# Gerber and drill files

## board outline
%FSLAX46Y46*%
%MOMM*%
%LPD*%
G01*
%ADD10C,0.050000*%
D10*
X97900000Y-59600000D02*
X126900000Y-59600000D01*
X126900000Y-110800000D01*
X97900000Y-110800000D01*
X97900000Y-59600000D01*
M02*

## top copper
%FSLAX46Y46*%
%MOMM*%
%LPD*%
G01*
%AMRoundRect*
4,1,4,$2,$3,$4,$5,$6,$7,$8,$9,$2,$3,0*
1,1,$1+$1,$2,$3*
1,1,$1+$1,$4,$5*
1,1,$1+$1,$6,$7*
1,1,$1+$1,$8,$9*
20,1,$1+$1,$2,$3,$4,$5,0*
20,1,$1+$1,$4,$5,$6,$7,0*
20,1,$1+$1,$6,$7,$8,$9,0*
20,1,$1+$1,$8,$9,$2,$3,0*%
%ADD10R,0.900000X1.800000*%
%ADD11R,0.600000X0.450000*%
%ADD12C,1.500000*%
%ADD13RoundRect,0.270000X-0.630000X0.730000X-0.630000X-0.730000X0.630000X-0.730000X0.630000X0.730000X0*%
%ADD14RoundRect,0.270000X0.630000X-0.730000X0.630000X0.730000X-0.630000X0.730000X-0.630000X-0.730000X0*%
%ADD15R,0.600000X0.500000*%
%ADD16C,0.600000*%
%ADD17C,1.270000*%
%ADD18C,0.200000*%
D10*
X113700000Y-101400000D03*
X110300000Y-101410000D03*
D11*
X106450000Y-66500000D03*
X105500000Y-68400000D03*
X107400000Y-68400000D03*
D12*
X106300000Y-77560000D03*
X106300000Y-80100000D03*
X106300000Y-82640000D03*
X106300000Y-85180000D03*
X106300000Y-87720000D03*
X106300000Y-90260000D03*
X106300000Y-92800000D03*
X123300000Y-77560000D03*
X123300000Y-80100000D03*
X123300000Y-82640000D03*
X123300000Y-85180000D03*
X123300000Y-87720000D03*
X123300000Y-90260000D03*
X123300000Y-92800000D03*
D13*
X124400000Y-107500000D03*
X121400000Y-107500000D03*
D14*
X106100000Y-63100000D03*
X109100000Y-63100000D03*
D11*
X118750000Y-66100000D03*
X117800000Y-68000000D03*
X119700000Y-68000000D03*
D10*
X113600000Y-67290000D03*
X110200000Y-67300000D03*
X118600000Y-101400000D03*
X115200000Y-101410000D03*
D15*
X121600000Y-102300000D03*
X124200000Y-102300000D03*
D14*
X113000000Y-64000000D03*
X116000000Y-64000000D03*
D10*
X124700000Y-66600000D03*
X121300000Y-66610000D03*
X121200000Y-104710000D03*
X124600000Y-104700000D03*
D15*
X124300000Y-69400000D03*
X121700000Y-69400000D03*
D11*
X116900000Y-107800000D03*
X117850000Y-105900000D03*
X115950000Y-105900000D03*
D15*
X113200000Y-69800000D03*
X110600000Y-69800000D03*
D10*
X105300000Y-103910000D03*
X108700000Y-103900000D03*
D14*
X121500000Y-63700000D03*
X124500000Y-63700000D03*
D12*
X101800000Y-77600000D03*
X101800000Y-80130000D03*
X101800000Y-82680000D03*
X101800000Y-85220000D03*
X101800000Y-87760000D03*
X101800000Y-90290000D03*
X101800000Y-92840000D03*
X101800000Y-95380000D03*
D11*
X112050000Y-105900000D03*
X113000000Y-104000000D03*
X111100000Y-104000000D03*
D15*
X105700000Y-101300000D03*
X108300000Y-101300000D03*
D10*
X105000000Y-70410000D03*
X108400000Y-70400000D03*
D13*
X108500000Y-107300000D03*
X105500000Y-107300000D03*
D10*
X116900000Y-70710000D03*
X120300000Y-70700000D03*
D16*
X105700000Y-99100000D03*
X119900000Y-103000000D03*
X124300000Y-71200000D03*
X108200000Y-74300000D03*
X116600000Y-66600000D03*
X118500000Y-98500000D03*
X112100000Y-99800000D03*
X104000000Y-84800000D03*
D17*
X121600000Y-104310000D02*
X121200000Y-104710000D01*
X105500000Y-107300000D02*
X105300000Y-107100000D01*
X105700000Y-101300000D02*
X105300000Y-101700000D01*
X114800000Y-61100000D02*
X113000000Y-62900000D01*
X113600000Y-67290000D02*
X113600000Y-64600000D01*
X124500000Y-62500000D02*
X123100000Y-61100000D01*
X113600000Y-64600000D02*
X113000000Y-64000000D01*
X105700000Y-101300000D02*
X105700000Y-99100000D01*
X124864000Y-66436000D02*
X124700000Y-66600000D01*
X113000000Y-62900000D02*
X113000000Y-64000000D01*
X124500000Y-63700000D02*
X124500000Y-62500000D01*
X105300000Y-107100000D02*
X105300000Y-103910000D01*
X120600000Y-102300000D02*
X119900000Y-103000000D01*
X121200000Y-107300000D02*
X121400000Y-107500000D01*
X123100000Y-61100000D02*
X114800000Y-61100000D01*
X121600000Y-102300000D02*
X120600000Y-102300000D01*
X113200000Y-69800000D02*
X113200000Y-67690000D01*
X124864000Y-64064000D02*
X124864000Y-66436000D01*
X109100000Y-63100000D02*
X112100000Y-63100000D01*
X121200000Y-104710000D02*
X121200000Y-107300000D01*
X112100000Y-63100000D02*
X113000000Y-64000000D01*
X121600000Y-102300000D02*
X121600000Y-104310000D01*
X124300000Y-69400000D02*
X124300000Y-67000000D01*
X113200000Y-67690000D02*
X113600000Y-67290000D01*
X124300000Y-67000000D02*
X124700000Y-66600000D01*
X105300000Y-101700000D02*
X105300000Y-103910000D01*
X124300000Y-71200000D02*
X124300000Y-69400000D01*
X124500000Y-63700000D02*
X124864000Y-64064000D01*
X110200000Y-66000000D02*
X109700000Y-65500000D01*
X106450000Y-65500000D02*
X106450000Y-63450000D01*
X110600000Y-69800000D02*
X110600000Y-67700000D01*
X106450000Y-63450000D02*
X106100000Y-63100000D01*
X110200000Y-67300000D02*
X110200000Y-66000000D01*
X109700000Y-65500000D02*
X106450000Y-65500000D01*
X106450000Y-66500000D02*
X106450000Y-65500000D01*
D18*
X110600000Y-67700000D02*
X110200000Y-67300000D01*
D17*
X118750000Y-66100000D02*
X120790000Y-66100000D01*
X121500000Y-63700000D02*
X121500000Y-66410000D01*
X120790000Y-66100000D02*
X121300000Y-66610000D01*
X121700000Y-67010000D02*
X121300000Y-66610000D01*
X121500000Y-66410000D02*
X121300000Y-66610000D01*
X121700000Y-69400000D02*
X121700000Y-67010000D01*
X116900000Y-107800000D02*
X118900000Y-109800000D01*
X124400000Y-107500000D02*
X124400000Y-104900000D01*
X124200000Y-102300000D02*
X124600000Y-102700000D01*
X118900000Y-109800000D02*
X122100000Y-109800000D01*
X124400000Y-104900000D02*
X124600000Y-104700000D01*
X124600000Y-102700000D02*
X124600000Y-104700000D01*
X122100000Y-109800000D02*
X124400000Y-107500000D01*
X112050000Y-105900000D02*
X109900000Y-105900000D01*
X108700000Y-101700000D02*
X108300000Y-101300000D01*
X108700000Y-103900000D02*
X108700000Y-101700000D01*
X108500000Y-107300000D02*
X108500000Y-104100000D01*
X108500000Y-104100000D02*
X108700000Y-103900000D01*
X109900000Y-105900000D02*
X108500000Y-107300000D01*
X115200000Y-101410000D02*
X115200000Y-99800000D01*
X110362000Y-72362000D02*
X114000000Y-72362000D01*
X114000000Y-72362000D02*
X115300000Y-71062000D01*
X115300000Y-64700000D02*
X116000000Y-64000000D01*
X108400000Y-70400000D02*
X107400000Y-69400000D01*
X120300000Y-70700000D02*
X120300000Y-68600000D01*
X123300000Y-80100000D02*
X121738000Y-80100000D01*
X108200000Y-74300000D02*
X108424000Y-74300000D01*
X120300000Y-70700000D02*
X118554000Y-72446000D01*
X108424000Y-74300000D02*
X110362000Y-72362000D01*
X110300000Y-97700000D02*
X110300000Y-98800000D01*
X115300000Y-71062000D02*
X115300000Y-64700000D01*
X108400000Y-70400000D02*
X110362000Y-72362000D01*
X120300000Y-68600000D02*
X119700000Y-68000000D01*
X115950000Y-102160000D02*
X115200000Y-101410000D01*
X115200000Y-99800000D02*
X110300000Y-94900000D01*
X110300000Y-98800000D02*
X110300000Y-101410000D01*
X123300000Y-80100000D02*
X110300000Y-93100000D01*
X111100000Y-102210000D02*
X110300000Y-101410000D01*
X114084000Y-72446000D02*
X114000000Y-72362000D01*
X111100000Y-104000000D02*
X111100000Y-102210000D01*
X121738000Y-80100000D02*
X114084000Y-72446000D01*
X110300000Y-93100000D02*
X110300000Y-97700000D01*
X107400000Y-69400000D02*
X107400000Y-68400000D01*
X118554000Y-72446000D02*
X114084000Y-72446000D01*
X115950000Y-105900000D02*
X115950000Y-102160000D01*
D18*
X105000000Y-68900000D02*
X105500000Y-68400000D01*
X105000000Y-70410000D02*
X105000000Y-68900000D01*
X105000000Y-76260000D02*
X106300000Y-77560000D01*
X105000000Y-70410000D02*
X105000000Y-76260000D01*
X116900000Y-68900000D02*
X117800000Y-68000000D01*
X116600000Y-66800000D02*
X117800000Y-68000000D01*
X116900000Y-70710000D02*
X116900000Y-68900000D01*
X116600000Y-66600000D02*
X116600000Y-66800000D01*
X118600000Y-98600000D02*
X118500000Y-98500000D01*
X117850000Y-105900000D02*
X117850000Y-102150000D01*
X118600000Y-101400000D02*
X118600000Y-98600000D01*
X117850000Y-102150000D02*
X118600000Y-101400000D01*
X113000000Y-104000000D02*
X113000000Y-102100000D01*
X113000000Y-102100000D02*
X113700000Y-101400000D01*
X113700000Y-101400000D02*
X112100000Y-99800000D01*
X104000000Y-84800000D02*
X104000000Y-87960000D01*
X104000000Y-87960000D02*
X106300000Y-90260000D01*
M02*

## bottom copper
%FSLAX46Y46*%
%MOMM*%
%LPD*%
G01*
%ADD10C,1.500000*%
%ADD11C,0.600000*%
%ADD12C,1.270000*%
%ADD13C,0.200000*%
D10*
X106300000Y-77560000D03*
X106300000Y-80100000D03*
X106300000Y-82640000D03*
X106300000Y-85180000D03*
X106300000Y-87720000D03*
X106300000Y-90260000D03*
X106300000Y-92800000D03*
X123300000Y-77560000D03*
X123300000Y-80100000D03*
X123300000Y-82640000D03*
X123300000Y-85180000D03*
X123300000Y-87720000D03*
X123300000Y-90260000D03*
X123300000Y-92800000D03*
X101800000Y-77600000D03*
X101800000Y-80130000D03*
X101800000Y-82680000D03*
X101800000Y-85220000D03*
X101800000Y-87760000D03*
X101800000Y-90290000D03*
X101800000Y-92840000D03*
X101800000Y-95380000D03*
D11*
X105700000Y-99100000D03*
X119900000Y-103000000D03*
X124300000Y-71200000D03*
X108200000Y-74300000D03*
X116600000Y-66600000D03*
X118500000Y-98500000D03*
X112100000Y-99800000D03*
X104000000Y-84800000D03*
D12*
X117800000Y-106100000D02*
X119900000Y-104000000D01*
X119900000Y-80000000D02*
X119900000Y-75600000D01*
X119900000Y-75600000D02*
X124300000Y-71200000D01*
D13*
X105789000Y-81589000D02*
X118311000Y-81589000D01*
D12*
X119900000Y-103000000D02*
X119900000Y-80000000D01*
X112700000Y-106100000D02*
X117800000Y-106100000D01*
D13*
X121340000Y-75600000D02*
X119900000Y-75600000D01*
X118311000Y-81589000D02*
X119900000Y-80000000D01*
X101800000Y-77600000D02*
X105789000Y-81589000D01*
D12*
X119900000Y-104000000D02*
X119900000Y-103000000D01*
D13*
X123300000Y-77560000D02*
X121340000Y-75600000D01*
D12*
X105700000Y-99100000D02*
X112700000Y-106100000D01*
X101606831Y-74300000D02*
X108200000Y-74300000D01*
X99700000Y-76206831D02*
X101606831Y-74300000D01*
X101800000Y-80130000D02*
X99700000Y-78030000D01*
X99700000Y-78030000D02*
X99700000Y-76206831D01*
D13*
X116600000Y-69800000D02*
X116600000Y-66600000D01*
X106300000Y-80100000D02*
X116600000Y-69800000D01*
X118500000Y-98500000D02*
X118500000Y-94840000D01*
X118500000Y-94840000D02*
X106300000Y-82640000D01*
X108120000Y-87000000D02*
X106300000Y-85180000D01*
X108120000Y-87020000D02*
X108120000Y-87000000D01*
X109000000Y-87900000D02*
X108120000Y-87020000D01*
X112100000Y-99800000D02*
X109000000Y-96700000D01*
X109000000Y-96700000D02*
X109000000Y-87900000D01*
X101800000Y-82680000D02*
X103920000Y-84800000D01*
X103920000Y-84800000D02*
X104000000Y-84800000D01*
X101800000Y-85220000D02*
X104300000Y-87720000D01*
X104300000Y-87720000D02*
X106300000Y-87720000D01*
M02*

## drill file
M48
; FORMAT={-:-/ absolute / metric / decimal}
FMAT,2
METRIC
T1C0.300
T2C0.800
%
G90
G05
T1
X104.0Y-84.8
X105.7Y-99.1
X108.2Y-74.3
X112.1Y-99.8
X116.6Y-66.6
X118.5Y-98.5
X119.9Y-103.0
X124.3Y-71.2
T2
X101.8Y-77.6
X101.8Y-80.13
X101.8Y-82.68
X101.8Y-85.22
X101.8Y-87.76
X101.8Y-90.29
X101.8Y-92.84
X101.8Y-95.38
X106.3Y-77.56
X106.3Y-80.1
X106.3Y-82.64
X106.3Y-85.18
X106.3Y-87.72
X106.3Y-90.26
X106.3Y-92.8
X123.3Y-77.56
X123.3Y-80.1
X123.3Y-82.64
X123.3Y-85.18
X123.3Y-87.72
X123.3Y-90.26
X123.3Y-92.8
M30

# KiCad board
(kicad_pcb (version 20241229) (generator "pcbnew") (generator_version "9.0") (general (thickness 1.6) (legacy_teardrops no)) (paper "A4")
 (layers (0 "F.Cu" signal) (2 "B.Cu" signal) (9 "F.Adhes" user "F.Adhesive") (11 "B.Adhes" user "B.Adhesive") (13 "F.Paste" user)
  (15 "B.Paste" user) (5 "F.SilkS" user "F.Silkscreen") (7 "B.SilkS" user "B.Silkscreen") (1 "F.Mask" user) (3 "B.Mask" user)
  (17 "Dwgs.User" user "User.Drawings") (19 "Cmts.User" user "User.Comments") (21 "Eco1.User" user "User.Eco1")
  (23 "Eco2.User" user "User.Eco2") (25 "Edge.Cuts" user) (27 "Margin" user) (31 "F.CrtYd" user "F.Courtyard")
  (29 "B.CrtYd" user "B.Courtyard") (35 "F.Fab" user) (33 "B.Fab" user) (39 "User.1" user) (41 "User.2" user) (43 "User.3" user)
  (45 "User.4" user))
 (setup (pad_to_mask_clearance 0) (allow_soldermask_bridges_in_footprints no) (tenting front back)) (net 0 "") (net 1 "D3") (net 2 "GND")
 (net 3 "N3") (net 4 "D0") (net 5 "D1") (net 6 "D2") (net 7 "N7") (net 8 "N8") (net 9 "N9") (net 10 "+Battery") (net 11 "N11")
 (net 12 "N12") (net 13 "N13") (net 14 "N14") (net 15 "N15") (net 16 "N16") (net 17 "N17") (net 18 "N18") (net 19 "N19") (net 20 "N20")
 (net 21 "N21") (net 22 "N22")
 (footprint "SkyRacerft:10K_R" (layer "F.Cu") (at 112 101.41 180)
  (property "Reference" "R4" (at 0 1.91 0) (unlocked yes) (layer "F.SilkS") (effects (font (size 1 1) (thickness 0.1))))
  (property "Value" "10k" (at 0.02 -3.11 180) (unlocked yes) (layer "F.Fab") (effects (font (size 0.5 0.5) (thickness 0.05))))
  (pad "1" smd rect (at -1.7 0.01 180) (size 0.9 1.8) (layers "F.Cu" "F.Mask" "F.Paste") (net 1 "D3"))
  (pad "2" smd rect (at 1.7 0 180) (size 0.9 1.8) (layers "F.Cu" "F.Mask" "F.Paste") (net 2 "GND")))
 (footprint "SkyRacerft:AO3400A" (layer "F.Cu") (at 106.45 67.45)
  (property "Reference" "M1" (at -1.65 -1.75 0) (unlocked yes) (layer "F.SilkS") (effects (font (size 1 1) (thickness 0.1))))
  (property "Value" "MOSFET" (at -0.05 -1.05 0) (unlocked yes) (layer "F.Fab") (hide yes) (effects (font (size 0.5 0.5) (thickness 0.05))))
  (pad "1" smd rect (at 0 -0.95 90) (size 0.45 0.6) (layers "F.Cu" "F.Mask" "F.Paste") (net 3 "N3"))
  (pad "2" smd rect (at -0.95 0.95 90) (size 0.45 0.6) (layers "F.Cu" "F.Mask" "F.Paste") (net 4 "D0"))
  (pad "3" smd rect (at 0.95 0.95 90) (size 0.45 0.6) (layers "F.Cu" "F.Mask" "F.Paste") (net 2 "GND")))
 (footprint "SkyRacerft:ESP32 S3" (layer "F.Cu") (at 114.8 77.56)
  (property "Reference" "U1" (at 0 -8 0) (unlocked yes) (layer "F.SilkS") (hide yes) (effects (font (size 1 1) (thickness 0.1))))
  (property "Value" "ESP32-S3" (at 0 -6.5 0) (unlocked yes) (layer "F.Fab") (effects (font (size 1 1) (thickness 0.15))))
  (pad "1" thru_hole circle (at -8.5 0) (size 1.5 1.5) (drill 0.8) (layers "*.Cu" "*.Mask") (remove_unused_layers no) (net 4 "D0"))
  (pad "2" thru_hole circle (at -8.5 2.54) (size 1.5 1.5) (drill 0.8) (layers "*.Cu" "*.Mask") (remove_unused_layers no) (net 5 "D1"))
  (pad "3" thru_hole circle (at -8.5 5.08) (size 1.5 1.5) (drill 0.8) (layers "*.Cu" "*.Mask") (remove_unused_layers no) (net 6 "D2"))
  (pad "4" thru_hole circle (at -8.5 7.62) (size 1.5 1.5) (drill 0.8) (layers "*.Cu" "*.Mask") (remove_unused_layers no) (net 1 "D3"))
  (pad "5" thru_hole circle (at -8.5 10.16) (size 1.5 1.5) (drill 0.8) (layers "*.Cu" "*.Mask") (remove_unused_layers no) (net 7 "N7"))
  (pad "6" thru_hole circle (at -8.5 12.7) (size 1.5 1.5) (drill 0.8) (layers "*.Cu" "*.Mask") (remove_unused_layers no) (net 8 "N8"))
  (pad "7" thru_hole circle (at -8.5 15.24) (size 1.5 1.5) (drill 0.8) (layers "*.Cu" "*.Mask") (remove_unused_layers no) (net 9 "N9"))
  (pad "8" thru_hole circle (at 8.5 0) (size 1.5 1.5) (drill 0.8) (layers "*.Cu" "*.Mask") (remove_unused_layers no) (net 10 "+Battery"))
  (pad "9" thru_hole circle (at 8.5 2.54) (size 1.5 1.5) (drill 0.8) (layers "*.Cu" "*.Mask") (remove_unused_layers no) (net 2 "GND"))
  (pad "10" thru_hole circle (at 8.5 5.08) (size 1.5 1.5) (drill 0.8) (layers "*.Cu" "*.Mask") (remove_unused_layers no) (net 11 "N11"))
  (pad "11" thru_hole circle (at 8.5 7.62) (size 1.5 1.5) (drill 0.8) (layers "*.Cu" "*.Mask") (remove_unused_layers no) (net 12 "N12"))
  (pad "12" thru_hole circle (at 8.5 10.16) (size 1.5 1.5) (drill 0.8) (layers "*.Cu" "*.Mask") (remove_unused_layers no) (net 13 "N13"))
  (pad "13" thru_hole circle (at 8.5 12.7) (size 1.5 1.5) (drill 0.8) (layers "*.Cu" "*.Mask") (remove_unused_layers no) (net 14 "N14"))
  (pad "14" thru_hole circle (at 8.5 15.24) (size 1.5 1.5) (drill 0.8) (layers "*.Cu" "*.Mask") (remove_unused_layers no) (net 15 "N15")))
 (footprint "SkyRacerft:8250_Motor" (layer "F.Cu") (at 122.9 107.5 180)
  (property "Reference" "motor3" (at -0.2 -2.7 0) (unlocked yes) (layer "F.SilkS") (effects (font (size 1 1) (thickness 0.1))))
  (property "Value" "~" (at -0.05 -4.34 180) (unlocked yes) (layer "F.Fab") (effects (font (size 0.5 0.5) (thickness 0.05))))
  (pad "1" smd roundrect (at -1.5 0 270) (size 2 1.8) (layers "F.Cu" "F.Mask" "F.Paste") (roundrect_rratio 0.15) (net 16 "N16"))
  (pad "2" smd roundrect (at 1.5 0 270) (size 2 1.8) (layers "F.Cu" "F.Mask" "F.Paste") (roundrect_rratio 0.15) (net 10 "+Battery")))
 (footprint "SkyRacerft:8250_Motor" (layer "F.Cu") (at 107.6 63.1)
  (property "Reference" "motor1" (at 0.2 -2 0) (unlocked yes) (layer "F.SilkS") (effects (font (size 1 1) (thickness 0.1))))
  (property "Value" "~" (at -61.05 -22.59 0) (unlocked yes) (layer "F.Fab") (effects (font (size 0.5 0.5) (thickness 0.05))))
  (pad "1" smd roundrect (at -1.5 0 90) (size 2 1.8) (layers "F.Cu" "F.Mask" "F.Paste") (roundrect_rratio 0.15) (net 3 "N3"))
  (pad "2" smd roundrect (at 1.5 0 90) (size 2 1.8) (layers "F.Cu" "F.Mask" "F.Paste") (roundrect_rratio 0.15) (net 10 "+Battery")))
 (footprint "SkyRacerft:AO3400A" (layer "F.Cu") (at 118.75 67.05)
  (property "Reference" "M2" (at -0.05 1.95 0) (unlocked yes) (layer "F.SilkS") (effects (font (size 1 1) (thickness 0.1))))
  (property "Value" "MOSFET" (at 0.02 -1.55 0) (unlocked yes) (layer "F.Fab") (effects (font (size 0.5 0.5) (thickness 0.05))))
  (pad "1" smd rect (at 0 -0.95 90) (size 0.45 0.6) (layers "F.Cu" "F.Mask" "F.Paste") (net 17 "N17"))
  (pad "2" smd rect (at -0.95 0.95 90) (size 0.45 0.6) (layers "F.Cu" "F.Mask" "F.Paste") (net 5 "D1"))
  (pad "3" smd rect (at 0.95 0.95 90) (size 0.45 0.6) (layers "F.Cu" "F.Mask" "F.Paste") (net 2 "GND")))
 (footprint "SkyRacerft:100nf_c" (layer "F.Cu") (at 111.9 67.3 180)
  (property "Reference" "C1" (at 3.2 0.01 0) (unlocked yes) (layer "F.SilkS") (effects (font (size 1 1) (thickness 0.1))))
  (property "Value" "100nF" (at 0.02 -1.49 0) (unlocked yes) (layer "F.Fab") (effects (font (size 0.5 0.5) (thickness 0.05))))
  (pad "1" smd rect (at -1.7 0.01 180) (size 0.9 1.8) (layers "F.Cu" "F.Mask" "F.Paste") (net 10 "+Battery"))
  (pad "2" smd rect (at 1.7 0 180) (size 0.9 1.8) (layers "F.Cu" "F.Mask" "F.Paste") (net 3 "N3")))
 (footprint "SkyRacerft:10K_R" (layer "F.Cu") (at 116.9 101.41 180)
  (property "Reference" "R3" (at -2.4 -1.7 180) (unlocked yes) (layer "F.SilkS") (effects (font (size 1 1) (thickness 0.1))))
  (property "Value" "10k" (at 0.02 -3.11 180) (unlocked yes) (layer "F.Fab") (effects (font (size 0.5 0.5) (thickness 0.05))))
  (pad "1" smd rect (at -1.7 0.01 180) (size 0.9 1.8) (layers "F.Cu" "F.Mask" "F.Paste") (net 6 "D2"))
  (pad "2" smd rect (at 1.7 0 180) (size 0.9 1.8) (layers "F.Cu" "F.Mask" "F.Paste") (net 2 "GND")))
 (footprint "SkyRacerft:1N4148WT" (layer "F.Cu") (at 122.9 102.3 180)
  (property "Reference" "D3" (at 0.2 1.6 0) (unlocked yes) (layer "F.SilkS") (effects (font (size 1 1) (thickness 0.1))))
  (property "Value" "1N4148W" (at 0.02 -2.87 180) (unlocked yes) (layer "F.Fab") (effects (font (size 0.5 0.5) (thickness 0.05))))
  (pad "1" smd rect (at 1.3 0 180) (size 0.6 0.5) (layers "F.Cu" "F.Mask" "F.Paste") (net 10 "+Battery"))
  (pad "2" smd rect (at -1.3 0 180) (size 0.6 0.5) (layers "F.Cu" "F.Mask" "F.Paste") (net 16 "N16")))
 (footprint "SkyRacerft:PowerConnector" (layer "F.Cu") (at 114.5 64)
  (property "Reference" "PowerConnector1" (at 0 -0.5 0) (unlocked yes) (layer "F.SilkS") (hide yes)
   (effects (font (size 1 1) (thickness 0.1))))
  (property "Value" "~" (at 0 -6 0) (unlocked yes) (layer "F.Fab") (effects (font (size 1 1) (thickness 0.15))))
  (pad "1" smd roundrect (at -1.5 0 90) (size 2 1.8) (layers "F.Cu" "F.Mask" "F.Paste") (roundrect_rratio 0.15) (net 10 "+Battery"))
  (pad "2" smd roundrect (at 1.5 0 90) (size 2 1.8) (layers "F.Cu" "F.Mask" "F.Paste") (roundrect_rratio 0.15) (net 2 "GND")))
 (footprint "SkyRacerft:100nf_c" (layer "F.Cu") (at 123 66.61 180)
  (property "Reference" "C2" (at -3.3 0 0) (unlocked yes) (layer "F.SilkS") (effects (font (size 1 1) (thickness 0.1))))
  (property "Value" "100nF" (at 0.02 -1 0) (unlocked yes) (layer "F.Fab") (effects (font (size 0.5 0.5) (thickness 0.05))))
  (pad "1" smd rect (at -1.7 0.01 180) (size 0.9 1.8) (layers "F.Cu" "F.Mask" "F.Paste") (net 10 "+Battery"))
  (pad "2" smd rect (at 1.7 0 180) (size 0.9 1.8) (layers "F.Cu" "F.Mask" "F.Paste") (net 17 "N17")))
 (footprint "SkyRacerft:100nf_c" (layer "F.Cu") (at 122.9 104.7)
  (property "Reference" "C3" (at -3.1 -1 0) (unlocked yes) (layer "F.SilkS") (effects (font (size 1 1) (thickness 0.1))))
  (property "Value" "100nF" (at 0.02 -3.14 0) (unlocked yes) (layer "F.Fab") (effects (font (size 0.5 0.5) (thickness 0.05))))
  (pad "1" smd rect (at -1.7 0.01) (size 0.9 1.8) (layers "F.Cu" "F.Mask" "F.Paste") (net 10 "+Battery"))
  (pad "2" smd rect (at 1.7 0) (size 0.9 1.8) (layers "F.Cu" "F.Mask" "F.Paste") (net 16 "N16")))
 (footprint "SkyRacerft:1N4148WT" (layer "F.Cu") (at 123 69.4)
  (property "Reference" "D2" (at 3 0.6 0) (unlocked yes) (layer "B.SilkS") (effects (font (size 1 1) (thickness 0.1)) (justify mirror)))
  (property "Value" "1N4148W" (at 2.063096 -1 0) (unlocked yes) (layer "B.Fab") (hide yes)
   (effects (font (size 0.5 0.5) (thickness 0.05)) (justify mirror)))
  (pad "1" smd rect (at 1.3 0) (size 0.6 0.5) (layers "F.Cu" "F.Mask" "F.Paste") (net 10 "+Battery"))
  (pad "2" smd rect (at -1.3 0) (size 0.6 0.5) (layers "F.Cu" "F.Mask" "F.Paste") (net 17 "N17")))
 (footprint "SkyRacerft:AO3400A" (layer "F.Cu") (at 116.9 106.85 180)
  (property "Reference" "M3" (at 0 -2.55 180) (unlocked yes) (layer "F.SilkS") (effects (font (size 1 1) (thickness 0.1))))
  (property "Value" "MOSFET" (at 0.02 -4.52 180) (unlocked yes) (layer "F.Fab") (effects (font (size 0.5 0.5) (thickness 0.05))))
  (pad "1" smd rect (at 0 -0.95 270) (size 0.45 0.6) (layers "F.Cu" "F.Mask" "F.Paste") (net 16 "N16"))
  (pad "2" smd rect (at -0.95 0.95 270) (size 0.45 0.6) (layers "F.Cu" "F.Mask" "F.Paste") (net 6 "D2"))
  (pad "3" smd rect (at 0.95 0.95 270) (size 0.45 0.6) (layers "F.Cu" "F.Mask" "F.Paste") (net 2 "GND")))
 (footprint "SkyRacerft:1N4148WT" (layer "F.Cu") (at 111.9 69.8)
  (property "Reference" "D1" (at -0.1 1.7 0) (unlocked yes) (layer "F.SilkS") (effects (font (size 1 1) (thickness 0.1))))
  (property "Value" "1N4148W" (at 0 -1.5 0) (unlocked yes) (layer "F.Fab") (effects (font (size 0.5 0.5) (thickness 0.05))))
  (pad "1" smd rect (at 1.3 0) (size 0.6 0.5) (layers "F.Cu" "F.Mask" "F.Paste") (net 10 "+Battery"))
  (pad "2" smd rect (at -1.3 0) (size 0.6 0.5) (layers "F.Cu" "F.Mask" "F.Paste") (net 3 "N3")))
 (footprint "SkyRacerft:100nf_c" (layer "F.Cu") (at 107 103.9)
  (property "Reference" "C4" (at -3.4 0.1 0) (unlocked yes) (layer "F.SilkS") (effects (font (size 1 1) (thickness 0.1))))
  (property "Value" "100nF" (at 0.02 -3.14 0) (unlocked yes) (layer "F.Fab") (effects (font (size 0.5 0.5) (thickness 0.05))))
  (pad "1" smd rect (at -1.7 0.01) (size 0.9 1.8) (layers "F.Cu" "F.Mask" "F.Paste") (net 10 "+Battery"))
  (pad "2" smd rect (at 1.7 0) (size 0.9 1.8) (layers "F.Cu" "F.Mask" "F.Paste") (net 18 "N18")))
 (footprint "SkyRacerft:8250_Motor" (layer "F.Cu") (at 123 63.7)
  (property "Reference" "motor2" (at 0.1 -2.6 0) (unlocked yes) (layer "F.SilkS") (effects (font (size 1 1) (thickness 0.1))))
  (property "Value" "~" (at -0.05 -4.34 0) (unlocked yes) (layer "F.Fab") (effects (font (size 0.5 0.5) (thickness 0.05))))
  (pad "1" smd roundrect (at -1.5 0 90) (size 2 1.8) (layers "F.Cu" "F.Mask" "F.Paste") (roundrect_rratio 0.15) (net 17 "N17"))
  (pad "2" smd roundrect (at 1.5 0 90) (size 2 1.8) (layers "F.Cu" "F.Mask" "F.Paste") (roundrect_rratio 0.15) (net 10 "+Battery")))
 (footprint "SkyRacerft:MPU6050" (layer "F.Cu") (at 101.8 77.6)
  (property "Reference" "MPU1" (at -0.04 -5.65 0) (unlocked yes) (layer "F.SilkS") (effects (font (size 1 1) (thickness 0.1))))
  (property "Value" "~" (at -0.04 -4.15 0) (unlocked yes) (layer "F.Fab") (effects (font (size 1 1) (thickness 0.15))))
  (pad "1" thru_hole circle (at 0 0) (size 1.5 1.5) (drill 0.8) (layers "*.Cu" "*.Mask") (remove_unused_layers no) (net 10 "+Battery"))
  (pad "2" thru_hole circle (at 0 2.53) (size 1.5 1.5) (drill 0.8) (layers "*.Cu" "*.Mask") (remove_unused_layers no) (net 2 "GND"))
  (pad "3" thru_hole circle (at 0 5.08) (size 1.5 1.5) (drill 0.8) (layers "*.Cu" "*.Mask") (remove_unused_layers no) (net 8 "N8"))
  (pad "4" thru_hole circle (at 0 7.62) (size 1.5 1.5) (drill 0.8) (layers "*.Cu" "*.Mask") (remove_unused_layers no) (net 7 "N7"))
  (pad "5" thru_hole circle (at 0 10.16) (size 1.5 1.5) (drill 0.8) (layers "*.Cu" "*.Mask") (remove_unused_layers no) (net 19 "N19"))
  (pad "6" thru_hole circle (at 0 12.69) (size 1.5 1.5) (drill 0.8) (layers "*.Cu" "*.Mask") (remove_unused_layers no) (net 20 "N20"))
  (pad "7" thru_hole circle (at 0 15.24) (size 1.5 1.5) (drill 0.8) (layers "*.Cu" "*.Mask") (remove_unused_layers no) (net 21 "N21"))
  (pad "8" thru_hole circle (at 0 17.78) (size 1.5 1.5) (drill 0.8) (layers "*.Cu" "*.Mask") (remove_unused_layers no) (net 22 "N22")))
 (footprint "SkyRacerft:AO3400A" (layer "F.Cu") (at 112.05 104.95 180)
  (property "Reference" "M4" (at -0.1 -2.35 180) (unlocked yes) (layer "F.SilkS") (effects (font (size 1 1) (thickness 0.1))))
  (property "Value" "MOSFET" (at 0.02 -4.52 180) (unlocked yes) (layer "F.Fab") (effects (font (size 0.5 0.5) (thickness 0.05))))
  (pad "1" smd rect (at 0 -0.95 270) (size 0.45 0.6) (layers "F.Cu" "F.Mask" "F.Paste") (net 18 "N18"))
  (pad "2" smd rect (at -0.95 0.95 270) (size 0.45 0.6) (layers "F.Cu" "F.Mask" "F.Paste") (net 1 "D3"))
  (pad "3" smd rect (at 0.95 0.95 270) (size 0.45 0.6) (layers "F.Cu" "F.Mask" "F.Paste") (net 2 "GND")))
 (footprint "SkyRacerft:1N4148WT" (layer "F.Cu") (at 107 101.3 180)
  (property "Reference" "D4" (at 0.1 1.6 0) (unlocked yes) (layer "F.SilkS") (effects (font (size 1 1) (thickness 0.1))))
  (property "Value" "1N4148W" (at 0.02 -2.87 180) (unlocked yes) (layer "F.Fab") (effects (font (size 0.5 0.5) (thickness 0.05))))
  (pad "1" smd rect (at 1.3 0 180) (size 0.6 0.5) (layers "F.Cu" "F.Mask" "F.Paste") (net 10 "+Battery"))
  (pad "2" smd rect (at -1.3 0 180) (size 0.6 0.5) (layers "F.Cu" "F.Mask" "F.Paste") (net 18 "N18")))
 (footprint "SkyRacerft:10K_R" (layer "F.Cu") (at 106.7 70.4)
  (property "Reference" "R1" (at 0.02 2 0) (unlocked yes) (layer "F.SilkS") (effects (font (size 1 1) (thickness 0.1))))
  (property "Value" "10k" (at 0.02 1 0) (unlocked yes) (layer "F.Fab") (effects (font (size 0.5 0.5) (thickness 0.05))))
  (pad "1" smd rect (at -1.7 0.01) (size 0.9 1.8) (layers "F.Cu" "F.Mask" "F.Paste") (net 4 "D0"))
  (pad "2" smd rect (at 1.7 0) (size 0.9 1.8) (layers "F.Cu" "F.Mask" "F.Paste") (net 2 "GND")))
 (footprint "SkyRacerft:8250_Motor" (layer "F.Cu") (at 107 107.3 180)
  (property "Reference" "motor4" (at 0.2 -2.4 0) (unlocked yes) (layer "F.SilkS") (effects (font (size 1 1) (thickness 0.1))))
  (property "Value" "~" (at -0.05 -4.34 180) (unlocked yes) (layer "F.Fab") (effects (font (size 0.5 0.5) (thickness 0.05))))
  (pad "1" smd roundrect (at -1.5 0 270) (size 2 1.8) (layers "F.Cu" "F.Mask" "F.Paste") (roundrect_rratio 0.15) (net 18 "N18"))
  (pad "2" smd roundrect (at 1.5 0 270) (size 2 1.8) (layers "F.Cu" "F.Mask" "F.Paste") (roundrect_rratio 0.15) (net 10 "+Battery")))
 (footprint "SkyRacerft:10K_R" (layer "F.Cu") (at 118.6 70.7)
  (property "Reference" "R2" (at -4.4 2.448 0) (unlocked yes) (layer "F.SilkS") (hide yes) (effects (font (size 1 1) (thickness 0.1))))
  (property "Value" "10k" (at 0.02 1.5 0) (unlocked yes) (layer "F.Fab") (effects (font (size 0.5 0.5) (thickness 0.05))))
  (pad "1" smd rect (at -1.7 0.01) (size 0.9 1.8) (layers "F.Cu" "F.Mask" "F.Paste") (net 5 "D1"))
  (pad "2" smd rect (at 1.7 0) (size 0.9 1.8) (layers "F.Cu" "F.Mask" "F.Paste") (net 2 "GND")))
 (gr_rect (start 97.9 59.6) (end 126.9 110.8) (stroke (width 0.05) (type default)) (fill no) (layer "Edge.Cuts"))
 (segment (start 121.6 104.31) (end 121.2 104.71) (width 1.27) (layer "F.Cu") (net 10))
 (segment (start 105.5 107.3) (end 105.3 107.1) (width 1.27) (layer "F.Cu") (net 10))
 (segment (start 105.7 101.3) (end 105.3 101.7) (width 1.27) (layer "F.Cu") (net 10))
 (segment (start 114.8 61.1) (end 113 62.9) (width 1.27) (layer "F.Cu") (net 10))
 (segment (start 113.6 67.29) (end 113.6 64.6) (width 1.27) (layer "F.Cu") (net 10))
 (segment (start 124.5 62.5) (end 123.1 61.1) (width 1.27) (layer "F.Cu") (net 10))
 (segment (start 113.6 64.6) (end 113 64) (width 1.27) (layer "F.Cu") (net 10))
 (segment (start 105.7 101.3) (end 105.7 99.1) (width 1.27) (layer "F.Cu") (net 10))
 (segment (start 124.864 66.436) (end 124.7 66.6) (width 1.27) (layer "F.Cu") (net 10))
 (segment (start 113 62.9) (end 113 64) (width 1.27) (layer "F.Cu") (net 10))
 (segment (start 124.5 63.7) (end 124.5 62.5) (width 1.27) (layer "F.Cu") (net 10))
 (segment (start 105.3 107.1) (end 105.3 103.91) (width 1.27) (layer "F.Cu") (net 10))
 (segment (start 120.6 102.3) (end 119.9 103) (width 1.27) (layer "F.Cu") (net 10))
 (segment (start 121.2 107.3) (end 121.4 107.5) (width 1.27) (layer "F.Cu") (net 10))
 (segment (start 123.1 61.1) (end 114.8 61.1) (width 1.27) (layer "F.Cu") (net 10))
 (segment (start 121.6 102.3) (end 120.6 102.3) (width 1.27) (layer "F.Cu") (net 10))
 (segment (start 113.2 69.8) (end 113.2 67.69) (width 1.27) (layer "F.Cu") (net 10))
 (segment (start 124.864 64.064) (end 124.864 66.436) (width 1.27) (layer "F.Cu") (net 10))
 (segment (start 109.1 63.1) (end 112.1 63.1) (width 1.27) (layer "F.Cu") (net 10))
 (segment (start 121.2 104.71) (end 121.2 107.3) (width 1.27) (layer "F.Cu") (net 10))
 (segment (start 112.1 63.1) (end 113 64) (width 1.27) (layer "F.Cu") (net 10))
 (segment (start 121.6 102.3) (end 121.6 104.31) (width 1.27) (layer "F.Cu") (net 10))
 (segment (start 124.3 69.4) (end 124.3 67) (width 1.27) (layer "F.Cu") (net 10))
 (segment (start 113.2 67.69) (end 113.6 67.29) (width 1.27) (layer "F.Cu") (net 10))
 (segment (start 124.3 67) (end 124.7 66.6) (width 1.27) (layer "F.Cu") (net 10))
 (segment (start 105.3 101.7) (end 105.3 103.91) (width 1.27) (layer "F.Cu") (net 10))
 (segment (start 124.3 71.2) (end 124.3 69.4) (width 1.27) (layer "F.Cu") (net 10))
 (segment (start 124.5 63.7) (end 124.864 64.064) (width 1.27) (layer "F.Cu") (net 10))
 (via (at 105.7 99.1) (size 0.6) (drill 0.3) (layers "F.Cu" "B.Cu") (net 10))
 (via (at 119.9 103) (size 0.6) (drill 0.3) (layers "F.Cu" "B.Cu") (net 10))
 (via (at 124.3 71.2) (size 0.6) (drill 0.3) (layers "F.Cu" "B.Cu") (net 10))
 (segment (start 117.8 106.1) (end 119.9 104) (width 1.27) (layer "B.Cu") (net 10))
 (segment (start 119.9 80) (end 119.9 75.6) (width 1.27) (layer "B.Cu") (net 10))
 (segment (start 119.9 75.6) (end 124.3 71.2) (width 1.27) (layer "B.Cu") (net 10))
 (segment (start 105.789 81.589) (end 118.311 81.589) (width 0.2) (layer "B.Cu") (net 10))
 (segment (start 119.9 103) (end 119.9 80) (width 1.27) (layer "B.Cu") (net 10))
 (segment (start 112.7 106.1) (end 117.8 106.1) (width 1.27) (layer "B.Cu") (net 10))
 (segment (start 121.34 75.6) (end 119.9 75.6) (width 0.2) (layer "B.Cu") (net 10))
 (segment (start 118.311 81.589) (end 119.9 80) (width 0.2) (layer "B.Cu") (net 10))
 (segment (start 101.8 77.6) (end 105.789 81.589) (width 0.2) (layer "B.Cu") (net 10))
 (segment (start 119.9 104) (end 119.9 103) (width 1.27) (layer "B.Cu") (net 10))
 (segment (start 123.3 77.56) (end 121.34 75.6) (width 0.2) (layer "B.Cu") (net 10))
 (segment (start 105.7 99.1) (end 112.7 106.1) (width 1.27) (layer "B.Cu") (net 10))
 (segment (start 110.2 66) (end 109.7 65.5) (width 1.27) (layer "F.Cu") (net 3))
 (segment (start 106.45 65.5) (end 106.45 63.45) (width 1.27) (layer "F.Cu") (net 3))
 (segment (start 110.6 69.8) (end 110.6 67.7) (width 1.27) (layer "F.Cu") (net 3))
 (segment (start 106.45 63.45) (end 106.1 63.1) (width 1.27) (layer "F.Cu") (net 3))
 (segment (start 110.2 67.3) (end 110.2 66) (width 1.27) (layer "F.Cu") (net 3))
 (segment (start 109.7 65.5) (end 106.45 65.5) (width 1.27) (layer "F.Cu") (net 3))
 (segment (start 106.45 66.5) (end 106.45 65.5) (width 1.27) (layer "F.Cu") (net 3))
 (segment (start 110.6 67.7) (end 110.2 67.3) (width 0.2) (layer "F.Cu") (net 3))
 (segment (start 118.75 66.1) (end 120.79 66.1) (width 1.27) (layer "F.Cu") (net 17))
 (segment (start 121.5 63.7) (end 121.5 66.41) (width 1.27) (layer "F.Cu") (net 17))
 (segment (start 120.79 66.1) (end 121.3 66.61) (width 1.27) (layer "F.Cu") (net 17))
 (segment (start 121.7 67.01) (end 121.3 66.61) (width 1.27) (layer "F.Cu") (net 17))
 (segment (start 121.5 66.41) (end 121.3 66.61) (width 1.27) (layer "F.Cu") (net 17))
 (segment (start 121.7 69.4) (end 121.7 67.01) (width 1.27) (layer "F.Cu") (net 17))
 (segment (start 116.9 107.8) (end 118.9 109.8) (width 1.27) (layer "F.Cu") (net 16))
 (segment (start 124.4 107.5) (end 124.4 104.9) (width 1.27) (layer "F.Cu") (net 16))
 (segment (start 124.2 102.3) (end 124.6 102.7) (width 1.27) (layer "F.Cu") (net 16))
 (segment (start 118.9 109.8) (end 122.1 109.8) (width 1.27) (layer "F.Cu") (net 16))
 (segment (start 124.4 104.9) (end 124.6 104.7) (width 1.27) (layer "F.Cu") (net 16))
 (segment (start 124.6 102.7) (end 124.6 104.7) (width 1.27) (layer "F.Cu") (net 16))
 (segment (start 122.1 109.8) (end 124.4 107.5) (width 1.27) (layer "F.Cu") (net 16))
 (segment (start 112.05 105.9) (end 109.9 105.9) (width 1.27) (layer "F.Cu") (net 18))
 (segment (start 108.7 101.7) (end 108.3 101.3) (width 1.27) (layer "F.Cu") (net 18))
 (segment (start 108.7 103.9) (end 108.7 101.7) (width 1.27) (layer "F.Cu") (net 18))
 (segment (start 108.5 107.3) (end 108.5 104.1) (width 1.27) (layer "F.Cu") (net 18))
 (segment (start 108.5 104.1) (end 108.7 103.9) (width 1.27) (layer "F.Cu") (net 18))
 (segment (start 109.9 105.9) (end 108.5 107.3) (width 1.27) (layer "F.Cu") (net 18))
 (segment (start 115.2 101.41) (end 115.2 99.8) (width 1.27) (layer "F.Cu") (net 2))
 (segment (start 110.362 72.362) (end 114 72.362) (width 1.27) (layer "F.Cu") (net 2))
 (segment (start 114 72.362) (end 115.3 71.062) (width 1.27) (layer "F.Cu") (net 2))
 (segment (start 115.3 64.7) (end 116 64) (width 1.27) (layer "F.Cu") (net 2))
 (segment (start 108.4 70.4) (end 107.4 69.4) (width 1.27) (layer "F.Cu") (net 2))
 (segment (start 120.3 70.7) (end 120.3 68.6) (width 1.27) (layer "F.Cu") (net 2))
 (segment (start 123.3 80.1) (end 121.738 80.1) (width 1.27) (layer "F.Cu") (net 2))
 (segment (start 108.2 74.3) (end 108.424 74.3) (width 1.27) (layer "F.Cu") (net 2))
 (segment (start 120.3 70.7) (end 118.554 72.446) (width 1.27) (layer "F.Cu") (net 2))
 (segment (start 108.424 74.3) (end 110.362 72.362) (width 1.27) (layer "F.Cu") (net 2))
 (segment (start 110.3 97.7) (end 110.3 98.8) (width 1.27) (layer "F.Cu") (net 2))
 (segment (start 115.3 71.062) (end 115.3 64.7) (width 1.27) (layer "F.Cu") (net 2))
 (segment (start 108.4 70.4) (end 110.362 72.362) (width 1.27) (layer "F.Cu") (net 2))
 (segment (start 120.3 68.6) (end 119.7 68) (width 1.27) (layer "F.Cu") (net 2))
 (segment (start 115.95 102.16) (end 115.2 101.41) (width 1.27) (layer "F.Cu") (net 2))
 (segment (start 115.2 99.8) (end 110.3 94.9) (width 1.27) (layer "F.Cu") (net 2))
 (segment (start 110.3 98.8) (end 110.3 101.41) (width 1.27) (layer "F.Cu") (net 2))
 (segment (start 123.3 80.1) (end 110.3 93.1) (width 1.27) (layer "F.Cu") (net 2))
 (segment (start 111.1 102.21) (end 110.3 101.41) (width 1.27) (layer "F.Cu") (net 2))
 (segment (start 114.084 72.446) (end 114 72.362) (width 1.27) (layer "F.Cu") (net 2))
 (segment (start 111.1 104) (end 111.1 102.21) (width 1.27) (layer "F.Cu") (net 2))
 (segment (start 121.738 80.1) (end 114.084 72.446) (width 1.27) (layer "F.Cu") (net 2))
 (segment (start 110.3 93.1) (end 110.3 97.7) (width 1.27) (layer "F.Cu") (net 2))
 (segment (start 107.4 69.4) (end 107.4 68.4) (width 1.27) (layer "F.Cu") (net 2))
 (segment (start 118.554 72.446) (end 114.084 72.446) (width 1.27) (layer "F.Cu") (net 2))
 (segment (start 115.95 105.9) (end 115.95 102.16) (width 1.27) (layer "F.Cu") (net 2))
 (via (at 108.2 74.3) (size 0.6) (drill 0.3) (layers "F.Cu" "B.Cu") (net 2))
 (segment (start 101.606831 74.3) (end 108.2 74.3) (width 1.27) (layer "B.Cu") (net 2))
 (segment (start 99.7 76.206831) (end 101.606831 74.3) (width 1.27) (layer "B.Cu") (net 2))
 (segment (start 101.8 80.13) (end 99.7 78.03) (width 1.27) (layer "B.Cu") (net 2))
 (segment (start 99.7 78.03) (end 99.7 76.206831) (width 1.27) (layer "B.Cu") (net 2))
 (segment (start 105 68.9) (end 105.5 68.4) (width 0.2) (layer "F.Cu") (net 4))
 (segment (start 105 70.41) (end 105 68.9) (width 0.2) (layer "F.Cu") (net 4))
 (segment (start 105 76.26) (end 106.3 77.56) (width 0.2) (layer "F.Cu") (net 4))
 (segment (start 105 70.41) (end 105 76.26) (width 0.2) (layer "F.Cu") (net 4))
 (segment (start 116.9 68.9) (end 117.8 68) (width 0.2) (layer "F.Cu") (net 5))
 (segment (start 116.6 66.8) (end 117.8 68) (width 0.2) (layer "F.Cu") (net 5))
 (segment (start 116.9 70.71) (end 116.9 68.9) (width 0.2) (layer "F.Cu") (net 5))
 (segment (start 116.6 66.6) (end 116.6 66.8) (width 0.2) (layer "F.Cu") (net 5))
 (via (at 116.6 66.6) (size 0.6) (drill 0.3) (layers "F.Cu" "B.Cu") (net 5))
 (segment (start 116.6 69.8) (end 116.6 66.6) (width 0.2) (layer "B.Cu") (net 5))
 (segment (start 106.3 80.1) (end 116.6 69.8) (width 0.2) (layer "B.Cu") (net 5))
 (segment (start 118.6 98.6) (end 118.5 98.5) (width 0.2) (layer "F.Cu") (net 6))
 (segment (start 117.85 105.9) (end 117.85 102.15) (width 0.2) (layer "F.Cu") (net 6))
 (segment (start 118.6 101.4) (end 118.6 98.6) (width 0.2) (layer "F.Cu") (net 6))
 (segment (start 117.85 102.15) (end 118.6 101.4) (width 0.2) (layer "F.Cu") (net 6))
 (via (at 118.5 98.5) (size 0.6) (drill 0.3) (layers "F.Cu" "B.Cu") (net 6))
 (segment (start 118.5 98.5) (end 118.5 94.84) (width 0.2) (layer "B.Cu") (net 6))
 (segment (start 118.5 94.84) (end 106.3 82.64) (width 0.2) (layer "B.Cu") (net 6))
 (segment (start 113 104) (end 113 102.1) (width 0.2) (layer "F.Cu") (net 1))
 (segment (start 113 102.1) (end 113.7 101.4) (width 0.2) (layer "F.Cu") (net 1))
 (segment (start 113.7 101.4) (end 112.1 99.8) (width 0.2) (layer "F.Cu") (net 1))
 (via (at 112.1 99.8) (size 0.6) (drill 0.3) (layers "F.Cu" "B.Cu") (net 1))
 (segment (start 108.12 87) (end 106.3 85.18) (width 0.2) (layer "B.Cu") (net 1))
 (segment (start 108.12 87.02) (end 108.12 87) (width 0.2) (layer "B.Cu") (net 1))
 (segment (start 109 87.9) (end 108.12 87.02) (width 0.2) (layer "B.Cu") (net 1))
 (segment (start 112.1 99.8) (end 109 96.7) (width 0.2) (layer "B.Cu") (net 1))
 (segment (start 109 96.7) (end 109 87.9) (width 0.2) (layer "B.Cu") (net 1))
 (segment (start 104 84.8) (end 104 87.96) (width 0.2) (layer "F.Cu") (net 8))
 (segment (start 104 87.96) (end 106.3 90.26) (width 0.2) (layer "F.Cu") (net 8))
 (via (at 104 84.8) (size 0.6) (drill 0.3) (layers "F.Cu" "B.Cu") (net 8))
 (segment (start 101.8 82.68) (end 103.92 84.8) (width 0.2) (layer "B.Cu") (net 8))
 (segment (start 103.92 84.8) (end 104 84.8) (width 0.2) (layer "B.Cu") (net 8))
 (segment (start 101.8 85.22) (end 104.3 87.72) (width 0.2) (layer "B.Cu") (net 7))
 (segment (start 104.3 87.72) (end 106.3 87.72) (width 0.2) (layer "B.Cu") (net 7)))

